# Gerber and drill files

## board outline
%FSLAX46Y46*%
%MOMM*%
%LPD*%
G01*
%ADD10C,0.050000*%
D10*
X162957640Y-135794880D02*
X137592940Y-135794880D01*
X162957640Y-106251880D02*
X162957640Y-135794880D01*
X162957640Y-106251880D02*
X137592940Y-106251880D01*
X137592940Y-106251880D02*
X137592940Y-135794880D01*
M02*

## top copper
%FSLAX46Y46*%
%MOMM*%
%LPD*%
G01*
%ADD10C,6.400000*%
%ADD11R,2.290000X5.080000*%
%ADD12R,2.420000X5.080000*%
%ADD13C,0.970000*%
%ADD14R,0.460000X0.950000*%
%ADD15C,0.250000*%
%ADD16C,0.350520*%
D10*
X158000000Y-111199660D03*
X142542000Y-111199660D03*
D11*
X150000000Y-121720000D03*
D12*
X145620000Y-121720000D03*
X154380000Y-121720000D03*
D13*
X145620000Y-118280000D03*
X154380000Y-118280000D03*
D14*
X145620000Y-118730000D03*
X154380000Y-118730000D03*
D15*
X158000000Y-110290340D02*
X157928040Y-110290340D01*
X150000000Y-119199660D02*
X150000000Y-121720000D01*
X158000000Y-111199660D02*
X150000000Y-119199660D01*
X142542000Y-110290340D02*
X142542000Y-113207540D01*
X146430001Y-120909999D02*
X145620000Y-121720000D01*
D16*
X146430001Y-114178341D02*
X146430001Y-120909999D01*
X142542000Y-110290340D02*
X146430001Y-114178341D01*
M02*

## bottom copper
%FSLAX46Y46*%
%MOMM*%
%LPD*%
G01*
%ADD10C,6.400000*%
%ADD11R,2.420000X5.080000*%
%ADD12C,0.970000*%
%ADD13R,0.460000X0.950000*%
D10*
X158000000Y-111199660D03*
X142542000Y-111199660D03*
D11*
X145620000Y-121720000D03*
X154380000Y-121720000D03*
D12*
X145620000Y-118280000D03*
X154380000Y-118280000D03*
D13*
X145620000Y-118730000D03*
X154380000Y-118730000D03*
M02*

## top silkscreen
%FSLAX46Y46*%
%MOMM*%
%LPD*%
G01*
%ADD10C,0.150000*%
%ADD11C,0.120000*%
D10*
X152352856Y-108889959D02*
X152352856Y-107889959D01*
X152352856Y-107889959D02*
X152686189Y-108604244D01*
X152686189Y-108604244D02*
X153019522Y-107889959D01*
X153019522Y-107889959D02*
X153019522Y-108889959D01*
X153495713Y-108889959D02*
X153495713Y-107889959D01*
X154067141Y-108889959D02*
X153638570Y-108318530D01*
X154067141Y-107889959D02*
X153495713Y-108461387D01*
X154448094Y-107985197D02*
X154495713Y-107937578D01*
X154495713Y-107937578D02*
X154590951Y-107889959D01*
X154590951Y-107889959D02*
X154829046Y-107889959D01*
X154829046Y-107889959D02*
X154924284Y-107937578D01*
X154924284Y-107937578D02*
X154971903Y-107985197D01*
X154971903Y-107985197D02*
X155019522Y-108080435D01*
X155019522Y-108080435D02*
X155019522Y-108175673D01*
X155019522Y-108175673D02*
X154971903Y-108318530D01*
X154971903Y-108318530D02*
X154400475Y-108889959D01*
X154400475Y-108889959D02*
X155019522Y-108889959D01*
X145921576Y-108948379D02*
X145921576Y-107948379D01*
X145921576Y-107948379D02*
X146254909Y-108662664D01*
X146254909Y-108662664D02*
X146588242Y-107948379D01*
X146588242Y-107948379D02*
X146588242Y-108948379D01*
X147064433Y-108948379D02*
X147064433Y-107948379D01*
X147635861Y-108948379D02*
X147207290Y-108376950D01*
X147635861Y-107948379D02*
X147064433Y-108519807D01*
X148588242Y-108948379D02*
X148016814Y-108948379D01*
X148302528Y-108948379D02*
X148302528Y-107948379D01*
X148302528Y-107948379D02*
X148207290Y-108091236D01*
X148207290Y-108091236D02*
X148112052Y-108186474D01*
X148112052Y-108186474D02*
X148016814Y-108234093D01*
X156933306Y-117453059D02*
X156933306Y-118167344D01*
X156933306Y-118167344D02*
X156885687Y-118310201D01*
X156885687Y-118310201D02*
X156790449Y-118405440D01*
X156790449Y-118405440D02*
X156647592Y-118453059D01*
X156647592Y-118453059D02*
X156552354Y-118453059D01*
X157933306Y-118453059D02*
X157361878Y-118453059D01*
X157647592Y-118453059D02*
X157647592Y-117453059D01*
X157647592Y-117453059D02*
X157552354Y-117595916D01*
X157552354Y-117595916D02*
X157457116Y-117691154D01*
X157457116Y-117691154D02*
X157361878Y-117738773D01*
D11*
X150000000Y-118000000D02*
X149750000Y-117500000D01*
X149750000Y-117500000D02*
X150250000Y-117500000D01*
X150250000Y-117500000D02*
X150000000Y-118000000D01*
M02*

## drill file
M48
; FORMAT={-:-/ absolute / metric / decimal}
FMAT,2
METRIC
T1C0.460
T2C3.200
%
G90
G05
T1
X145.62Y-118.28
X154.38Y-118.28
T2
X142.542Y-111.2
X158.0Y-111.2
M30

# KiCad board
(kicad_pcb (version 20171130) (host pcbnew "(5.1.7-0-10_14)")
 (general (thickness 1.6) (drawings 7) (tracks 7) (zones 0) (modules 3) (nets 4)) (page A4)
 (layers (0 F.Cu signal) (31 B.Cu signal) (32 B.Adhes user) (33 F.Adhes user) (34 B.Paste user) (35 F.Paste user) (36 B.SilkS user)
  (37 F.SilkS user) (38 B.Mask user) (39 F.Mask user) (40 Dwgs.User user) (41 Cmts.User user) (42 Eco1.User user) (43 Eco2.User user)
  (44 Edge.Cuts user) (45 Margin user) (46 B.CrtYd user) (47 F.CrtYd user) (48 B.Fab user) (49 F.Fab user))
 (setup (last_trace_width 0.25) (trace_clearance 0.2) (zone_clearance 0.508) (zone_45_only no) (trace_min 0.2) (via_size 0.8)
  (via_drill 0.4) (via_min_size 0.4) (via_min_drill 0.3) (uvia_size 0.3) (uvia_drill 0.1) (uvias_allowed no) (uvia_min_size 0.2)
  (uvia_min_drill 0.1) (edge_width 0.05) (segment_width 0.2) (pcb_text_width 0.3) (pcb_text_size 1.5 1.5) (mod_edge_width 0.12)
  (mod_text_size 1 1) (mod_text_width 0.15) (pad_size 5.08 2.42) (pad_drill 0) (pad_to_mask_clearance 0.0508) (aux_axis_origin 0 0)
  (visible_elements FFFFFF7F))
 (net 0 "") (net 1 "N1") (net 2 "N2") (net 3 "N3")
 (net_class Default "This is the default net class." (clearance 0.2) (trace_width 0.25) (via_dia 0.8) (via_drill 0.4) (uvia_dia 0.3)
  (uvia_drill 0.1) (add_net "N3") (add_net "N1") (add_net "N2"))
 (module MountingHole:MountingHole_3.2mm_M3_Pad (layer F.Cu) (at 158 111.19966)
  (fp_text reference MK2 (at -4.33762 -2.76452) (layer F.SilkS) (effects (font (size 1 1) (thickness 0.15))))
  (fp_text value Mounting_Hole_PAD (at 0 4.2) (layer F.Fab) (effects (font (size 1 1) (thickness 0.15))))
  (pad 1 thru_hole circle (at 0 0) (size 6.4 6.4) (drill 3.2) (layers *.Cu *.Mask) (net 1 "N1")))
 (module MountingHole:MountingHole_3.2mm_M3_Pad (layer F.Cu) (at 142.542 111.19966)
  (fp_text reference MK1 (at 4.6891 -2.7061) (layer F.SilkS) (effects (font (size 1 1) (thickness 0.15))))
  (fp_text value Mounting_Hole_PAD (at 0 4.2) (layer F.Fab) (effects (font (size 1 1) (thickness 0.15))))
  (pad 1 thru_hole circle (at 0 0) (size 6.4 6.4) (drill 3.2) (layers *.Cu *.Mask) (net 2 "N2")))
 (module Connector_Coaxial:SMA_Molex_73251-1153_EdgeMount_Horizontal (layer F.Cu) (at 150 120 90)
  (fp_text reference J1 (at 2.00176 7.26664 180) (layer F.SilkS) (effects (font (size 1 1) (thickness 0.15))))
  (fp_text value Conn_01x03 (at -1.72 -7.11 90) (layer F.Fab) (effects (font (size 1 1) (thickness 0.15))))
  (fp_line (start 2 0) (end 2.5 -0.25) (layer F.SilkS) (width 0.12))
  (fp_line (start 2.5 -0.25) (end 2.5 0.25) (layer F.SilkS) (width 0.12))
  (fp_line (start 2.5 0.25) (end 2 0) (layer F.SilkS) (width 0.12))
  (pad 2 smd rect (at -1.72 0 90) (size 5.08 2.29) (layers F.Cu F.Paste F.Mask) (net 1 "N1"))
  (pad 3 smd rect (at -1.72 -4.38 90) (size 5.08 2.42) (layers F.Cu F.Paste F.Mask) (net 2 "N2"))
  (pad 1 smd rect (at -1.72 4.38 90) (size 5.08 2.42) (layers F.Cu F.Paste F.Mask) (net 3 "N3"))
  (pad 2 smd rect (at -1.72 -4.38 90) (size 5.08 2.42) (layers B.Cu B.Paste B.Mask) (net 1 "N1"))
  (pad 2 smd rect (at -1.72 4.38 90) (size 5.08 2.42) (layers B.Cu B.Paste B.Mask) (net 1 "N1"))
  (pad 2 thru_hole circle (at 1.72 -4.38 90) (size 0.97 0.97) (drill 0.46) (layers *.Cu) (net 1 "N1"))
  (pad 2 thru_hole circle (at 1.72 4.38 90) (size 0.97 0.97) (drill 0.46) (layers *.Cu) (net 1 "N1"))
  (pad 2 smd rect (at 1.27 -4.38 90) (size 0.95 0.46) (layers F.Cu) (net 1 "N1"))
  (pad 2 smd rect (at 1.27 4.38 90) (size 0.95 0.46) (layers F.Cu) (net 1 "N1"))
  (pad 2 smd rect (at 1.27 -4.38 90) (size 0.95 0.46) (layers B.Cu) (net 1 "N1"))
  (pad 2 smd rect (at 1.27 4.38 90) (size 0.95 0.46) (layers B.Cu) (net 1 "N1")))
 (gr_line (start 162.95764 135.79488) (end 137.59294 135.79488) (layer Edge.Cuts) (width 0.05))
 (gr_line (start 162.95764 106.25188) (end 162.95764 135.79488) (layer Edge.Cuts) (width 0.05))
 (gr_line (start 162.95764 106.25188) (end 137.59294 106.25188) (layer Edge.Cuts) (width 0.05))
 (gr_line (start 137.59294 106.25188) (end 137.59294 135.79488) (layer Edge.Cuts) (width 0.05))
 (segment (start 158 110.29034) (end 157.92804 110.29034) (width 0.25) (layer F.Cu) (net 1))
 (segment (start 150 119.19966) (end 150 121.72) (width 0.25) (layer F.Cu) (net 1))
 (segment (start 158 111.19966) (end 150 119.19966) (width 0.25) (layer F.Cu) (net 1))
 (segment (start 142.542 110.29034) (end 142.542 113.20754) (width 0.25) (layer F.Cu) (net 2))
 (segment (start 146.430001 120.909999) (end 145.62 121.72) (width 0.25) (layer F.Cu) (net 2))
 (segment (start 146.430001 114.178341) (end 146.430001 120.909999) (width 0.35052) (layer F.Cu) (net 2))
 (segment (start 142.542 110.29034) (end 146.430001 114.178341) (width 0.35052) (layer F.Cu) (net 2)))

